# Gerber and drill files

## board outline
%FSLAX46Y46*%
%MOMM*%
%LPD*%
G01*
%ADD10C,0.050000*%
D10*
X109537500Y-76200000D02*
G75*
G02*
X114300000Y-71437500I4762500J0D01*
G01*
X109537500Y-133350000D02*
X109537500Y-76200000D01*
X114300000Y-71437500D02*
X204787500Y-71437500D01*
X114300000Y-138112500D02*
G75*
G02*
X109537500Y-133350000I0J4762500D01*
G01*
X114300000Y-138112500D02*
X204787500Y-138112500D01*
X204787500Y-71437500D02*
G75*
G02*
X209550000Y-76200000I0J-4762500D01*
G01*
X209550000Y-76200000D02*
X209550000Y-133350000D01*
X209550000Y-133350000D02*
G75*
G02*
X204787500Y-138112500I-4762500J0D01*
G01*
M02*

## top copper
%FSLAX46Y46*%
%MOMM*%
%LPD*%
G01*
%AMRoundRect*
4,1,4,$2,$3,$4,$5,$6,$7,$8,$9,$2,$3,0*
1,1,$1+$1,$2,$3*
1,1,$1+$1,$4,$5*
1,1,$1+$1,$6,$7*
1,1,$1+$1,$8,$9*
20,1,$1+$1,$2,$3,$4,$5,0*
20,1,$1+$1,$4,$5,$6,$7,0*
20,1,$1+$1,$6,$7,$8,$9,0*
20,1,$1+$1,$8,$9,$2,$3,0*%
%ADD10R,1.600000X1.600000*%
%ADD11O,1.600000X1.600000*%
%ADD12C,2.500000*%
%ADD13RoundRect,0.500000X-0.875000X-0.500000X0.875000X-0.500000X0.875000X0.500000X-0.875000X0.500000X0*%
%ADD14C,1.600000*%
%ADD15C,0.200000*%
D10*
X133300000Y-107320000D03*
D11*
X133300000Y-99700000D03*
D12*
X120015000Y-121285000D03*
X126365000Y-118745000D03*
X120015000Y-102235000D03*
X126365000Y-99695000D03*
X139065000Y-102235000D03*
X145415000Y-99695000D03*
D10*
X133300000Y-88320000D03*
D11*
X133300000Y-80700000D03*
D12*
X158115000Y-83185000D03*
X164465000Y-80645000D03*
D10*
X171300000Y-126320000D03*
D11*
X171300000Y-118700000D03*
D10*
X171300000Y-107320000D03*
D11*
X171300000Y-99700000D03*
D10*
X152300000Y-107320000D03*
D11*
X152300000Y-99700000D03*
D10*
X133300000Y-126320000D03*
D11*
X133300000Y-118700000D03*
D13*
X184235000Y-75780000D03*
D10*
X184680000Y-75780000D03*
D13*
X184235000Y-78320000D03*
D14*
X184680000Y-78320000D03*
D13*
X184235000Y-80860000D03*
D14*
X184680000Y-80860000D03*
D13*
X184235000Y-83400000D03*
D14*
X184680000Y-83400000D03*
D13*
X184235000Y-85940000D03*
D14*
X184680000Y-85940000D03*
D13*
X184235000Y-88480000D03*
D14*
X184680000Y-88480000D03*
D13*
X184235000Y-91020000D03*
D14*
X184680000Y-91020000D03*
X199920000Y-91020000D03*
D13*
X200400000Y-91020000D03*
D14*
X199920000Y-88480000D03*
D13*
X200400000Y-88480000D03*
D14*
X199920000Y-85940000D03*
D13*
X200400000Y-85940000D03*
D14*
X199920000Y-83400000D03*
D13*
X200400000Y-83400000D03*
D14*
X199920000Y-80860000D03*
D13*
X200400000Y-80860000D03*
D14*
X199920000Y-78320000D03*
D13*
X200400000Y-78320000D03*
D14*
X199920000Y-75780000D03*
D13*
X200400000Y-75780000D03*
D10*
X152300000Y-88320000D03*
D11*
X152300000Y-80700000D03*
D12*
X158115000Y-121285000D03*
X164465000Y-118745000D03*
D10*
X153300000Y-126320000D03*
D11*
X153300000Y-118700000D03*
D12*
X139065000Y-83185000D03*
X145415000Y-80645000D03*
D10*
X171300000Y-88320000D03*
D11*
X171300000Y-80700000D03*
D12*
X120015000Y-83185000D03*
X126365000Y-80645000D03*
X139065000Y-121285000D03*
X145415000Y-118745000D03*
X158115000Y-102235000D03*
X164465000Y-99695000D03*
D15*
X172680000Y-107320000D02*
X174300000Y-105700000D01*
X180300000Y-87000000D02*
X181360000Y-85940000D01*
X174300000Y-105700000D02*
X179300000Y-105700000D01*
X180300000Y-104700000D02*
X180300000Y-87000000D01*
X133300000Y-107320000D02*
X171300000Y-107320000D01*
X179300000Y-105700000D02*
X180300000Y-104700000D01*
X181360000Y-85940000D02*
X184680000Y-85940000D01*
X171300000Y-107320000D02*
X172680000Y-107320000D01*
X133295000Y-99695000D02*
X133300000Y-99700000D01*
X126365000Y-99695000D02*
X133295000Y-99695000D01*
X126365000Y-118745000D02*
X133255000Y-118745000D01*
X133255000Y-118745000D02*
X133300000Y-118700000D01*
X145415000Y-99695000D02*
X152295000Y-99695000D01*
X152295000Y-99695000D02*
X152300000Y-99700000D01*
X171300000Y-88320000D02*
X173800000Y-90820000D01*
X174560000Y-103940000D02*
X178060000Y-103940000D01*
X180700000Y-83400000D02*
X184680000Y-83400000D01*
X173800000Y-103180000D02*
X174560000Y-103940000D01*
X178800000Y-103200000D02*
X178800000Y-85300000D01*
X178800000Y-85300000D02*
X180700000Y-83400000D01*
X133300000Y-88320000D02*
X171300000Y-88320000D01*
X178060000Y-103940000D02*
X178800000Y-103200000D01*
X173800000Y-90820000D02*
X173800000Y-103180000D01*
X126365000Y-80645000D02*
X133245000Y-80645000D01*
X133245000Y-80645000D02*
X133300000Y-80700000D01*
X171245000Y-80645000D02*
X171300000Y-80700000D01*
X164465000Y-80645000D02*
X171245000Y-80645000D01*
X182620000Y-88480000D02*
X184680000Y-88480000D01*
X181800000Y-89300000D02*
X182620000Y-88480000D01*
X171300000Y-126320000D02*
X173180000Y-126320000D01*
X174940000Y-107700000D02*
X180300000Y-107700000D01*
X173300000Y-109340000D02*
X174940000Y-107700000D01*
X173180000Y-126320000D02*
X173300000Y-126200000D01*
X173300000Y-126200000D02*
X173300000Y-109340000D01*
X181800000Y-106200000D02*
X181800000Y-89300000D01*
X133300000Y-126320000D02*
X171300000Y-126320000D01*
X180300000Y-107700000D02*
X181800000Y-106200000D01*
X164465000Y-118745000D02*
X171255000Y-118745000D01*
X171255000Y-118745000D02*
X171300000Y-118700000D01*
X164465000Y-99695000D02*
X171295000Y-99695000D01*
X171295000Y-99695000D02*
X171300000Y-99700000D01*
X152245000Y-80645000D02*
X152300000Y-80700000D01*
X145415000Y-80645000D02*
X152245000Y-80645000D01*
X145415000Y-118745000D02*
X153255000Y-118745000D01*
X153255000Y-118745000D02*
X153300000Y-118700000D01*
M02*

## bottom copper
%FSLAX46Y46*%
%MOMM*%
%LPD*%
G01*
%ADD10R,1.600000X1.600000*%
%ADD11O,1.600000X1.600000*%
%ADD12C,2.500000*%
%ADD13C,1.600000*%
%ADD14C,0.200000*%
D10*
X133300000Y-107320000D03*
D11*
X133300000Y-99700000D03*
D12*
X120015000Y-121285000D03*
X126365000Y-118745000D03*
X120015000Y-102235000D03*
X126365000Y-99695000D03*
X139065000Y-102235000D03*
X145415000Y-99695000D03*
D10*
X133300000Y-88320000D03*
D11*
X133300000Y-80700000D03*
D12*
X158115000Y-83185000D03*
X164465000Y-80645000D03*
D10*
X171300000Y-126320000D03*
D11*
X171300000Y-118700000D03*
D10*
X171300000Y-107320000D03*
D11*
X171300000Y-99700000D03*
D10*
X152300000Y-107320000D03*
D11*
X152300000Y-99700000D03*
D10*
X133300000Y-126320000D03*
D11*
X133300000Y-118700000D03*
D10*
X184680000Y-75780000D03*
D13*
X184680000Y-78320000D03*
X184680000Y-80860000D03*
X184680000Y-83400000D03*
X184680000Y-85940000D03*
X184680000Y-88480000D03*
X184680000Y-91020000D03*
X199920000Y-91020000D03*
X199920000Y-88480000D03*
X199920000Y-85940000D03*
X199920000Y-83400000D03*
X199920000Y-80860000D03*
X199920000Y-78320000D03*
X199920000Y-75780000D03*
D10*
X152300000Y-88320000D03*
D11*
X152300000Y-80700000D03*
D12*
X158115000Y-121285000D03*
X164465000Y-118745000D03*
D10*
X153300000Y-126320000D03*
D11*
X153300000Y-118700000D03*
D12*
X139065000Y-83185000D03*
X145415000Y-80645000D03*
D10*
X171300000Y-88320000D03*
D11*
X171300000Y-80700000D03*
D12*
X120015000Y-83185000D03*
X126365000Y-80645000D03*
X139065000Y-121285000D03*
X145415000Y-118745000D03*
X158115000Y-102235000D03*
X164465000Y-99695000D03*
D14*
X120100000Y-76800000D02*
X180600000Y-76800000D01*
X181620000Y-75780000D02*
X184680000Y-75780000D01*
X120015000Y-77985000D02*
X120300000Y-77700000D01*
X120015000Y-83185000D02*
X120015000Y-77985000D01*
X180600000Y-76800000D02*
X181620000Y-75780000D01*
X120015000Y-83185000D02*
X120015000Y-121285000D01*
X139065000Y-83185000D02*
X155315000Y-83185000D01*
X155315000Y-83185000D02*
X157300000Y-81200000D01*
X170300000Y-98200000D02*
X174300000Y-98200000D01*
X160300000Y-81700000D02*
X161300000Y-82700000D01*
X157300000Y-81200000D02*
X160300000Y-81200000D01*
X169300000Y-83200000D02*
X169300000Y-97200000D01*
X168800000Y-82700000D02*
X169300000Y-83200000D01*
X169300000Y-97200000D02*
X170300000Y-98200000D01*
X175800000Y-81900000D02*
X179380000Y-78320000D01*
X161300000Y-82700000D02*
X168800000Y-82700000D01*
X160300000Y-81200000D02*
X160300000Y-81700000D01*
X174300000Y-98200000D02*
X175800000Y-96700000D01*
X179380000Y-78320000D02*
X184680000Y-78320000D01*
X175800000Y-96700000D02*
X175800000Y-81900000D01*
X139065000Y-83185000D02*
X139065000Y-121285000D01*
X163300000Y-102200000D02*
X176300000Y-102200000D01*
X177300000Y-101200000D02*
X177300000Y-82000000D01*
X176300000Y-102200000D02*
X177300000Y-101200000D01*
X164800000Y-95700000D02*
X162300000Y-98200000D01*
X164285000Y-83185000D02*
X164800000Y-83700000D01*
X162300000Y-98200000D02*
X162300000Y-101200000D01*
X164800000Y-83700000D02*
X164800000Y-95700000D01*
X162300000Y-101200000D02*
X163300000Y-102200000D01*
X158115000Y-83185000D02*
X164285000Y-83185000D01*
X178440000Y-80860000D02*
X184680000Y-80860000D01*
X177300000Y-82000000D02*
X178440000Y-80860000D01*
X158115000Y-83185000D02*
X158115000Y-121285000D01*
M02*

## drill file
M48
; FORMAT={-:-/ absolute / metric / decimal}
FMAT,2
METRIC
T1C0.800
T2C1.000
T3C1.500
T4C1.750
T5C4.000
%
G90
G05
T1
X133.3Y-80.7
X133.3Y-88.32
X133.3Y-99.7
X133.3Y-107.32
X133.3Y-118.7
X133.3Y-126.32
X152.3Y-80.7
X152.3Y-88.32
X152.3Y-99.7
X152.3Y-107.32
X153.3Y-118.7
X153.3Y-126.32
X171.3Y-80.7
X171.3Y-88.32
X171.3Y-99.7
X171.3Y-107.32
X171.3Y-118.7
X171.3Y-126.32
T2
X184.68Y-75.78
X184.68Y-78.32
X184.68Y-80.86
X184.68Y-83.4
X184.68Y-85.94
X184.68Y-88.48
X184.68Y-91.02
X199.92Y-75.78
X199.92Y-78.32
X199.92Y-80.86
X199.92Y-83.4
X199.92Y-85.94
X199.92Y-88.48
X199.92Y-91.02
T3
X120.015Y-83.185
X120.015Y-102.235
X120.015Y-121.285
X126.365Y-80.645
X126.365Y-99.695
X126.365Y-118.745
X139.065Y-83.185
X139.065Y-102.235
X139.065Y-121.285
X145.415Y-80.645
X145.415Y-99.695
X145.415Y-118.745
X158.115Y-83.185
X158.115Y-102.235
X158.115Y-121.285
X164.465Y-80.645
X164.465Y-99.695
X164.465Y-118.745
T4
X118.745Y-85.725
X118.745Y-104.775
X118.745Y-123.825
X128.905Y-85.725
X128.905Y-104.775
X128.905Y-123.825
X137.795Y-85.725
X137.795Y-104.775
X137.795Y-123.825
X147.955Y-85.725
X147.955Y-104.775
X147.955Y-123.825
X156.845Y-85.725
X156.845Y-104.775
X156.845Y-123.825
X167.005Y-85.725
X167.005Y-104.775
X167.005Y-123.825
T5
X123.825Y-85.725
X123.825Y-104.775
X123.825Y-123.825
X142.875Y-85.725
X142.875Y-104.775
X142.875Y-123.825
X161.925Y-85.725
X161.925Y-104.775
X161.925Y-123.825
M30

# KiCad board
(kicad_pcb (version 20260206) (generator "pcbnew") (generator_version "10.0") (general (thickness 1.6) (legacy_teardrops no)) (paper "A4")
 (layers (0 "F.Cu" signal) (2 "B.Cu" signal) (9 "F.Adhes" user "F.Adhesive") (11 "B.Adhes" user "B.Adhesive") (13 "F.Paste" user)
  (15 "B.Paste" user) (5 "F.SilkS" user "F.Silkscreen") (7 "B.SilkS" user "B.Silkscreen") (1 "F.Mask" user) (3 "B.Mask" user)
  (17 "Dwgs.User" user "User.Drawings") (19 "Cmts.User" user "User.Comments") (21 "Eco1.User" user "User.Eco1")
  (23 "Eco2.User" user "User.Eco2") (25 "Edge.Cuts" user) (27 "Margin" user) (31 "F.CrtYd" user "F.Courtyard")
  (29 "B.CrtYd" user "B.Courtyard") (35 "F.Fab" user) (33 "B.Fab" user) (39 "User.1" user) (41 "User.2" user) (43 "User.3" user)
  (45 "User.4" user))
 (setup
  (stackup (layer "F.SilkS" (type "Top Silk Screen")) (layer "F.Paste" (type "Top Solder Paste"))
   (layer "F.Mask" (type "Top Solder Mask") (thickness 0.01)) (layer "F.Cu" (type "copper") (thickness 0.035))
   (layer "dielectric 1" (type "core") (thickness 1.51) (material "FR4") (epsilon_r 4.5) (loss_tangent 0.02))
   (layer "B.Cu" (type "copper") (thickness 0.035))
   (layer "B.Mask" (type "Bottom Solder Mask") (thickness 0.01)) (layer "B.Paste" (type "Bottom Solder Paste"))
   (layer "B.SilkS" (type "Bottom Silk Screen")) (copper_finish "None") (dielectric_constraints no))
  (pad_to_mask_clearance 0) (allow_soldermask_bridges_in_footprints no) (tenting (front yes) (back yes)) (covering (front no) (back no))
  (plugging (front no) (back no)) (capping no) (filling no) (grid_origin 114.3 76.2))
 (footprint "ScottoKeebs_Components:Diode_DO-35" (layer "F.Cu") (at 133.3 107.32 90)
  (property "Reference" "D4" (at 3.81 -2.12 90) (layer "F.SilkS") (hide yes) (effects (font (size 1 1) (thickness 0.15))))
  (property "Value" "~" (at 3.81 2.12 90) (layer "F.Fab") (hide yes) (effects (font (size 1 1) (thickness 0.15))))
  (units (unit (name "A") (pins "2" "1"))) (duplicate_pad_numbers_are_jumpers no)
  (pad "1" thru_hole rect (at 0 0 90) (size 1.6 1.6) (drill 0.8) (layers "*.Cu" "*.Mask") (remove_unused_layers no) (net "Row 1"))
  (pad "2" thru_hole oval (at 7.62 0 90) (size 1.6 1.6) (drill 0.8) (layers "*.Cu" "*.Mask") (remove_unused_layers no) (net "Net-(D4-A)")))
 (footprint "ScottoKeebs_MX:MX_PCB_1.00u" (layer "F.Cu") (at 123.825 123.825)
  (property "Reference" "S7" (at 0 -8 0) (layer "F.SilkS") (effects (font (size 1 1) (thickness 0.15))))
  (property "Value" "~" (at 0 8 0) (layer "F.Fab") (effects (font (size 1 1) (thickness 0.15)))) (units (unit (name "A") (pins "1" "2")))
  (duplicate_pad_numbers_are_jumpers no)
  (pad "" np_thru_hole circle (at -5.08 0) (size 1.75 1.75) (drill 1.75) (layers "*.Cu" "*.Mask"))
  (pad "" np_thru_hole circle (at 0 0) (size 4 4) (drill 4) (layers "*.Cu" "*.Mask"))
  (pad "" np_thru_hole circle (at 5.08 0) (size 1.75 1.75) (drill 1.75) (layers "*.Cu" "*.Mask"))
  (pad "1" thru_hole circle (at -3.81 -2.54) (size 2.5 2.5) (drill 1.5) (layers "*.Cu" "*.Mask") (remove_unused_layers no) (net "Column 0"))
  (pad "2" thru_hole circle (at 2.54 -5.08) (size 2.5 2.5) (drill 1.5) (layers "*.Cu" "*.Mask") (remove_unused_layers no) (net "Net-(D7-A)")))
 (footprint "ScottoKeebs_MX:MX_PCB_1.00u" (layer "F.Cu") (at 123.825 104.775)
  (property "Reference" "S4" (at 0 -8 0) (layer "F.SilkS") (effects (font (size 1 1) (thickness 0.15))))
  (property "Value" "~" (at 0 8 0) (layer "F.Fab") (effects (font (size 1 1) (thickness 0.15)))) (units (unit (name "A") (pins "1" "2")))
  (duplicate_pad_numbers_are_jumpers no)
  (pad "" np_thru_hole circle (at -5.08 0) (size 1.75 1.75) (drill 1.75) (layers "*.Cu" "*.Mask"))
  (pad "" np_thru_hole circle (at 0 0) (size 4 4) (drill 4) (layers "*.Cu" "*.Mask"))
  (pad "" np_thru_hole circle (at 5.08 0) (size 1.75 1.75) (drill 1.75) (layers "*.Cu" "*.Mask"))
  (pad "1" thru_hole circle (at -3.81 -2.54) (size 2.5 2.5) (drill 1.5) (layers "*.Cu" "*.Mask") (remove_unused_layers no) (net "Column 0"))
  (pad "2" thru_hole circle (at 2.54 -5.08) (size 2.5 2.5) (drill 1.5) (layers "*.Cu" "*.Mask") (remove_unused_layers no) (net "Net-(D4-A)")))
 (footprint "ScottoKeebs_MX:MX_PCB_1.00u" (layer "F.Cu") (at 142.875 104.775)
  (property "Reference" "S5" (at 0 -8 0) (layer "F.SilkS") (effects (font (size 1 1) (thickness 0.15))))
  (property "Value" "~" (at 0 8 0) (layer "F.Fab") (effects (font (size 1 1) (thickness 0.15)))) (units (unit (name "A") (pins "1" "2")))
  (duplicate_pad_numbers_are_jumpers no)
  (pad "" np_thru_hole circle (at -5.08 0) (size 1.75 1.75) (drill 1.75) (layers "*.Cu" "*.Mask"))
  (pad "" np_thru_hole circle (at 0 0) (size 4 4) (drill 4) (layers "*.Cu" "*.Mask"))
  (pad "" np_thru_hole circle (at 5.08 0) (size 1.75 1.75) (drill 1.75) (layers "*.Cu" "*.Mask"))
  (pad "1" thru_hole circle (at -3.81 -2.54) (size 2.5 2.5) (drill 1.5) (layers "*.Cu" "*.Mask") (remove_unused_layers no) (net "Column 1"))
  (pad "2" thru_hole circle (at 2.54 -5.08) (size 2.5 2.5) (drill 1.5) (layers "*.Cu" "*.Mask") (remove_unused_layers no) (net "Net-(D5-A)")))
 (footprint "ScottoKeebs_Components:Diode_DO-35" (layer "F.Cu") (at 133.3 88.32 90)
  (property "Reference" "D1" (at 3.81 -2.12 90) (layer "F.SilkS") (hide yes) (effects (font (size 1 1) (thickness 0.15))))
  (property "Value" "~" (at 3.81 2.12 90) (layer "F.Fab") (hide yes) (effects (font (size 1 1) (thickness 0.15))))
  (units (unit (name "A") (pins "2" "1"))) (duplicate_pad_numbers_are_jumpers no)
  (pad "1" thru_hole rect (at 0 0 90) (size 1.6 1.6) (drill 0.8) (layers "*.Cu" "*.Mask") (remove_unused_layers no) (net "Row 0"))
  (pad "2" thru_hole oval (at 7.62 0 90) (size 1.6 1.6) (drill 0.8) (layers "*.Cu" "*.Mask") (remove_unused_layers no) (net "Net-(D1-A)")))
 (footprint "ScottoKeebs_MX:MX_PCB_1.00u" (layer "F.Cu") (at 161.925 85.725)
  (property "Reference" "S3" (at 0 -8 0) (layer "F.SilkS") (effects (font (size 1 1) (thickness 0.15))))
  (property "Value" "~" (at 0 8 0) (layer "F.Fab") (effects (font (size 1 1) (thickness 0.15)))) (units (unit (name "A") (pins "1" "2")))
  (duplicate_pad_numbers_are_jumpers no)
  (pad "" np_thru_hole circle (at -5.08 0) (size 1.75 1.75) (drill 1.75) (layers "*.Cu" "*.Mask"))
  (pad "" np_thru_hole circle (at 0 0) (size 4 4) (drill 4) (layers "*.Cu" "*.Mask"))
  (pad "" np_thru_hole circle (at 5.08 0) (size 1.75 1.75) (drill 1.75) (layers "*.Cu" "*.Mask"))
  (pad "1" thru_hole circle (at -3.81 -2.54) (size 2.5 2.5) (drill 1.5) (layers "*.Cu" "*.Mask") (remove_unused_layers no) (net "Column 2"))
  (pad "2" thru_hole circle (at 2.54 -5.08) (size 2.5 2.5) (drill 1.5) (layers "*.Cu" "*.Mask") (remove_unused_layers no) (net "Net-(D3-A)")))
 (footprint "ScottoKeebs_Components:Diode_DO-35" (layer "F.Cu") (at 171.3 126.32 90)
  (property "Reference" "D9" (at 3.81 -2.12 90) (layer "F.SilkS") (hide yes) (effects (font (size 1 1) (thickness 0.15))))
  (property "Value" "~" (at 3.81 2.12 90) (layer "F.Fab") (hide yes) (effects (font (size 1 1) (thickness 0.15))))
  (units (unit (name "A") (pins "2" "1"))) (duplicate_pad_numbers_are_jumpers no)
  (pad "1" thru_hole rect (at 0 0 90) (size 1.6 1.6) (drill 0.8) (layers "*.Cu" "*.Mask") (remove_unused_layers no) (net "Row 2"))
  (pad "2" thru_hole oval (at 7.62 0 90) (size 1.6 1.6) (drill 0.8) (layers "*.Cu" "*.Mask") (remove_unused_layers no) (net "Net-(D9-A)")))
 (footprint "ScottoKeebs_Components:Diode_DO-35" (layer "F.Cu") (at 171.3 107.32 90)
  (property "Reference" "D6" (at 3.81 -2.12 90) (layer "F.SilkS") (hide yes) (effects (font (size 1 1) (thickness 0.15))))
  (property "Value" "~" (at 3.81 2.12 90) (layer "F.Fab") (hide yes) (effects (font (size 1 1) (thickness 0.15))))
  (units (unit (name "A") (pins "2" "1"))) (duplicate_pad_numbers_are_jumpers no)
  (pad "1" thru_hole rect (at 0 0 90) (size 1.6 1.6) (drill 0.8) (layers "*.Cu" "*.Mask") (remove_unused_layers no) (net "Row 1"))
  (pad "2" thru_hole oval (at 7.62 0 90) (size 1.6 1.6) (drill 0.8) (layers "*.Cu" "*.Mask") (remove_unused_layers no) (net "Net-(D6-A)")))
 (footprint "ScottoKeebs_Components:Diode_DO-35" (layer "F.Cu") (at 152.3 107.32 90)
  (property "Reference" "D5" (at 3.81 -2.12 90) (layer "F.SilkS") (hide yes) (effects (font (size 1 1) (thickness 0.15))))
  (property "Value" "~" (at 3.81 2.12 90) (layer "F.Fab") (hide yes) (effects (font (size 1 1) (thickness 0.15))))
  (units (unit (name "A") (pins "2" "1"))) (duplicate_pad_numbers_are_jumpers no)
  (pad "1" thru_hole rect (at 0 0 90) (size 1.6 1.6) (drill 0.8) (layers "*.Cu" "*.Mask") (remove_unused_layers no) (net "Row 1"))
  (pad "2" thru_hole oval (at 7.62 0 90) (size 1.6 1.6) (drill 0.8) (layers "*.Cu" "*.Mask") (remove_unused_layers no) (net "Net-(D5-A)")))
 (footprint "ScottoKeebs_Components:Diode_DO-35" (layer "F.Cu") (at 133.3 126.32 90)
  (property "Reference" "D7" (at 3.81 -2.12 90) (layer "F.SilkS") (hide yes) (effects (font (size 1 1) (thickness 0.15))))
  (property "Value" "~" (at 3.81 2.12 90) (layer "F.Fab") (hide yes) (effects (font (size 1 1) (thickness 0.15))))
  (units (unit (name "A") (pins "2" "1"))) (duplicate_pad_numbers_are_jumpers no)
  (pad "1" thru_hole rect (at 0 0 90) (size 1.6 1.6) (drill 0.8) (layers "*.Cu" "*.Mask") (remove_unused_layers no) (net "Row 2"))
  (pad "2" thru_hole oval (at 7.62 0 90) (size 1.6 1.6) (drill 0.8) (layers "*.Cu" "*.Mask") (remove_unused_layers no) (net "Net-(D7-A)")))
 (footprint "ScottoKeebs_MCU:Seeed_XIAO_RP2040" (layer "F.Cu") (at 192.3 83.4)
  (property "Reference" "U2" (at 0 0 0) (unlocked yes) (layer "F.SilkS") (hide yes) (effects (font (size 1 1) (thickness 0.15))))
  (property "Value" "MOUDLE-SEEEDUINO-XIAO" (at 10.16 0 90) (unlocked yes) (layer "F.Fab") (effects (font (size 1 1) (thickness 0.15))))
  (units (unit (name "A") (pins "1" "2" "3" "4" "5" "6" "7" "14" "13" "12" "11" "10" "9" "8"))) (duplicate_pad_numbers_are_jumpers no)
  (pad "1" smd roundrect (at -8.065 -7.62) (size 2.75 2) (layers "F.Cu" "F.Mask" "F.Paste") (roundrect_rratio 0.25) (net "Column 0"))
  (pad "1" thru_hole rect (at -7.62 -7.62 90) (size 1.6 1.6) (drill 1) (layers "*.Cu" "*.Mask") (remove_unused_layers no) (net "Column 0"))
  (pad "2" smd roundrect (at -8.065 -5.08) (size 2.75 2) (layers "F.Cu" "F.Mask" "F.Paste") (roundrect_rratio 0.25) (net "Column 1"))
  (pad "2" thru_hole circle (at -7.62 -5.08 90) (size 1.6 1.6) (drill 1) (layers "*.Cu" "*.Mask") (remove_unused_layers no) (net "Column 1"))
  (pad "3" smd roundrect (at -8.065 -2.54) (size 2.75 2) (layers "F.Cu" "F.Mask" "F.Paste") (roundrect_rratio 0.25) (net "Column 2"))
  (pad "3" thru_hole circle (at -7.62 -2.54 90) (size 1.6 1.6) (drill 1) (layers "*.Cu" "*.Mask") (remove_unused_layers no) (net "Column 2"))
  (pad "4" smd roundrect (at -8.065 0) (size 2.75 2) (layers "F.Cu" "F.Mask" "F.Paste") (roundrect_rratio 0.25) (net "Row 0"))
  (pad "4" thru_hole circle (at -7.62 0 90) (size 1.6 1.6) (drill 1) (layers "*.Cu" "*.Mask") (remove_unused_layers no) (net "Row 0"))
  (pad "5" smd roundrect (at -8.065 2.54) (size 2.75 2) (layers "F.Cu" "F.Mask" "F.Paste") (roundrect_rratio 0.25) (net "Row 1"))
  (pad "5" thru_hole circle (at -7.62 2.54 90) (size 1.6 1.6) (drill 1) (layers "*.Cu" "*.Mask") (remove_unused_layers no) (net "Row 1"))
  (pad "6" smd roundrect (at -8.065 5.08) (size 2.75 2) (layers "F.Cu" "F.Mask" "F.Paste") (roundrect_rratio 0.25) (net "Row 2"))
  (pad "6" thru_hole circle (at -7.62 5.08 90) (size 1.6 1.6) (drill 1) (layers "*.Cu" "*.Mask") (remove_unused_layers no) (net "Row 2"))
  (pad "7" smd roundrect (at -8.065 7.62) (size 2.75 2) (layers "F.Cu" "F.Mask" "F.Paste") (roundrect_rratio 0.25)
   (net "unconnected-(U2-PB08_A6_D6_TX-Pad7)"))
  (pad "7" thru_hole circle (at -7.62 7.62 90) (size 1.6 1.6) (drill 1) (layers "*.Cu" "*.Mask") (remove_unused_layers no)
   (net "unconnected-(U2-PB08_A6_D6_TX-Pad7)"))
  (pad "8" thru_hole circle (at 7.62 7.62 90) (size 1.6 1.6) (drill 1) (layers "*.Cu" "*.Mask") (remove_unused_layers no)
   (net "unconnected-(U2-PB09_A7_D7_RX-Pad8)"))
  (pad "8" smd roundrect (at 8.1 7.62) (size 2.75 2) (layers "F.Cu" "F.Mask" "F.Paste") (roundrect_rratio 0.25)
   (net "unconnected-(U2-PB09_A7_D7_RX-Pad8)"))
  (pad "9" thru_hole circle (at 7.62 5.08 90) (size 1.6 1.6) (drill 1) (layers "*.Cu" "*.Mask") (remove_unused_layers no)
   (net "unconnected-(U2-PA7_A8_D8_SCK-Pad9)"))
  (pad "9" smd roundrect (at 8.1 5.08) (size 2.75 2) (layers "F.Cu" "F.Mask" "F.Paste") (roundrect_rratio 0.25)
   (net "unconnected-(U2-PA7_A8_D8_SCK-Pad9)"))
  (pad "10" thru_hole circle (at 7.62 2.54 90) (size 1.6 1.6) (drill 1) (layers "*.Cu" "*.Mask") (remove_unused_layers no)
   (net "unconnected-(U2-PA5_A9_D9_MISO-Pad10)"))
  (pad "10" smd roundrect (at 8.1 2.54) (size 2.75 2) (layers "F.Cu" "F.Mask" "F.Paste") (roundrect_rratio 0.25)
   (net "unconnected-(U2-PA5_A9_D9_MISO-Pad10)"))
  (pad "11" thru_hole circle (at 7.62 0 90) (size 1.6 1.6) (drill 1) (layers "*.Cu" "*.Mask") (remove_unused_layers no)
   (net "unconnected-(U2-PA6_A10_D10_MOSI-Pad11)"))
  (pad "11" smd roundrect (at 8.1 0) (size 2.75 2) (layers "F.Cu" "F.Mask" "F.Paste") (roundrect_rratio 0.25)
   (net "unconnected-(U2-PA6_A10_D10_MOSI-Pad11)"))
  (pad "12" thru_hole circle (at 7.62 -2.54 90) (size 1.6 1.6) (drill 1) (layers "*.Cu" "*.Mask") (remove_unused_layers no)
   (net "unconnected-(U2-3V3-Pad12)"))
  (pad "12" smd roundrect (at 8.1 -2.54) (size 2.75 2) (layers "F.Cu" "F.Mask" "F.Paste") (roundrect_rratio 0.25)
   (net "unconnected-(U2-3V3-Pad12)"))
  (pad "13" thru_hole circle (at 7.62 -5.08 90) (size 1.6 1.6) (drill 1) (layers "*.Cu" "*.Mask") (remove_unused_layers no)
   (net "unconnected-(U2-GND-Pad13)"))
  (pad "13" smd roundrect (at 8.1 -5.08) (size 2.75 2) (layers "F.Cu" "F.Mask" "F.Paste") (roundrect_rratio 0.25)
   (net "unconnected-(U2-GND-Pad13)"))
  (pad "14" thru_hole circle (at 7.62 -7.62 90) (size 1.6 1.6) (drill 1) (layers "*.Cu" "*.Mask") (remove_unused_layers no)
   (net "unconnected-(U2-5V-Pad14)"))
  (pad "14" smd roundrect (at 8.1 -7.62) (size 2.75 2) (layers "F.Cu" "F.Mask" "F.Paste") (roundrect_rratio 0.25)
   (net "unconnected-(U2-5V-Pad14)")))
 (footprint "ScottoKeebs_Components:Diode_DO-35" (layer "F.Cu") (at 152.3 88.32 90)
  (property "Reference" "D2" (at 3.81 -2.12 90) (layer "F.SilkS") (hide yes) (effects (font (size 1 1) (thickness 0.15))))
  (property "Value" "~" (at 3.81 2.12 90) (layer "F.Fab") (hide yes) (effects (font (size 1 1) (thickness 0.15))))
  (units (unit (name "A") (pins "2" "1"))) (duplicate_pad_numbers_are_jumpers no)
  (pad "1" thru_hole rect (at 0 0 90) (size 1.6 1.6) (drill 0.8) (layers "*.Cu" "*.Mask") (remove_unused_layers no) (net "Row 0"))
  (pad "2" thru_hole oval (at 7.62 0 90) (size 1.6 1.6) (drill 0.8) (layers "*.Cu" "*.Mask") (remove_unused_layers no) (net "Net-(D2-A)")))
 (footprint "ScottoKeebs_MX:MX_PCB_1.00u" (layer "F.Cu") (at 161.925 123.825)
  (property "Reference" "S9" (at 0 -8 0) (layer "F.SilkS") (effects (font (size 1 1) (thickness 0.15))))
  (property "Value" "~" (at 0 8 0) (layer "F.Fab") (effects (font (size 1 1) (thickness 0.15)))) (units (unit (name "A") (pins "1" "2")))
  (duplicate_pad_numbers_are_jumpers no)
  (pad "" np_thru_hole circle (at -5.08 0) (size 1.75 1.75) (drill 1.75) (layers "*.Cu" "*.Mask"))
  (pad "" np_thru_hole circle (at 0 0) (size 4 4) (drill 4) (layers "*.Cu" "*.Mask"))
  (pad "" np_thru_hole circle (at 5.08 0) (size 1.75 1.75) (drill 1.75) (layers "*.Cu" "*.Mask"))
  (pad "1" thru_hole circle (at -3.81 -2.54) (size 2.5 2.5) (drill 1.5) (layers "*.Cu" "*.Mask") (remove_unused_layers no) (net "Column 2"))
  (pad "2" thru_hole circle (at 2.54 -5.08) (size 2.5 2.5) (drill 1.5) (layers "*.Cu" "*.Mask") (remove_unused_layers no) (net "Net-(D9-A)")))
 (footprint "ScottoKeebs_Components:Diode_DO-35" (layer "F.Cu") (at 153.3 126.32 90)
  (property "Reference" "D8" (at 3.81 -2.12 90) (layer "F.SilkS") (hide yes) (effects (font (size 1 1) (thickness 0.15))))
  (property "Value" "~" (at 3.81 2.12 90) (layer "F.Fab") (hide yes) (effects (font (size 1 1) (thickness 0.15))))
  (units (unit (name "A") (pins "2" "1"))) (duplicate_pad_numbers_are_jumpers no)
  (pad "1" thru_hole rect (at 0 0 90) (size 1.6 1.6) (drill 0.8) (layers "*.Cu" "*.Mask") (remove_unused_layers no) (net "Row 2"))
  (pad "2" thru_hole oval (at 7.62 0 90) (size 1.6 1.6) (drill 0.8) (layers "*.Cu" "*.Mask") (remove_unused_layers no) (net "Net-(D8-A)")))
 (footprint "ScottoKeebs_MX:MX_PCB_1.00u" (layer "F.Cu") (at 142.875 85.725)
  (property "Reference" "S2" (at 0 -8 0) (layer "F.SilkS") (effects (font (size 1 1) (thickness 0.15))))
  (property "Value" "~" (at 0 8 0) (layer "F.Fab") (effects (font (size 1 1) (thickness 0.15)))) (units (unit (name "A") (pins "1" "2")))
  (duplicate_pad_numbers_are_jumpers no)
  (pad "" np_thru_hole circle (at -5.08 0) (size 1.75 1.75) (drill 1.75) (layers "*.Cu" "*.Mask"))
  (pad "" np_thru_hole circle (at 0 0) (size 4 4) (drill 4) (layers "*.Cu" "*.Mask"))
  (pad "" np_thru_hole circle (at 5.08 0) (size 1.75 1.75) (drill 1.75) (layers "*.Cu" "*.Mask"))
  (pad "1" thru_hole circle (at -3.81 -2.54) (size 2.5 2.5) (drill 1.5) (layers "*.Cu" "*.Mask") (remove_unused_layers no) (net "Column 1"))
  (pad "2" thru_hole circle (at 2.54 -5.08) (size 2.5 2.5) (drill 1.5) (layers "*.Cu" "*.Mask") (remove_unused_layers no) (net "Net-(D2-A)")))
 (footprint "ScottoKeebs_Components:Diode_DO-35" (layer "F.Cu") (at 171.3 88.32 90)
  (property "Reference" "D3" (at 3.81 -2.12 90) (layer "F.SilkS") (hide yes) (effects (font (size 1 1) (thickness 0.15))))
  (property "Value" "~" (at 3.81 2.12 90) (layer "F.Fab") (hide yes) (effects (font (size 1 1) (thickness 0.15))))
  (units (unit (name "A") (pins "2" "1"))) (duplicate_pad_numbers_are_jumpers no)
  (pad "1" thru_hole rect (at 0 0 90) (size 1.6 1.6) (drill 0.8) (layers "*.Cu" "*.Mask") (remove_unused_layers no) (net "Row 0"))
  (pad "2" thru_hole oval (at 7.62 0 90) (size 1.6 1.6) (drill 0.8) (layers "*.Cu" "*.Mask") (remove_unused_layers no) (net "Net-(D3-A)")))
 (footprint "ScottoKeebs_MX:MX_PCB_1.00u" (layer "F.Cu") (at 123.825 85.725)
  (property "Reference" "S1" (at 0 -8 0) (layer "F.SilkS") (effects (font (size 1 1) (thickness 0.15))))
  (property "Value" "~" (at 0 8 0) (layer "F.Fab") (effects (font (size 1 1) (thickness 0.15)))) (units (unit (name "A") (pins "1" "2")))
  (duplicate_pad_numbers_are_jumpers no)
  (pad "" np_thru_hole circle (at -5.08 0) (size 1.75 1.75) (drill 1.75) (layers "*.Cu" "*.Mask"))
  (pad "" np_thru_hole circle (at 0 0) (size 4 4) (drill 4) (layers "*.Cu" "*.Mask"))
  (pad "" np_thru_hole circle (at 5.08 0) (size 1.75 1.75) (drill 1.75) (layers "*.Cu" "*.Mask"))
  (pad "1" thru_hole circle (at -3.81 -2.54) (size 2.5 2.5) (drill 1.5) (layers "*.Cu" "*.Mask") (remove_unused_layers no) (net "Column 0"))
  (pad "2" thru_hole circle (at 2.54 -5.08) (size 2.5 2.5) (drill 1.5) (layers "*.Cu" "*.Mask") (remove_unused_layers no) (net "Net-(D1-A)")))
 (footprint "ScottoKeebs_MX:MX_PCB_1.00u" (layer "F.Cu") (at 142.875 123.825)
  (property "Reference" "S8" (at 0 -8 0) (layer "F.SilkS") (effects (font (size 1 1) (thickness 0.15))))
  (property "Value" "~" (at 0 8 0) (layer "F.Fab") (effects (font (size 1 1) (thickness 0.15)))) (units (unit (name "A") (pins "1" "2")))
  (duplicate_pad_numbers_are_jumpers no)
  (pad "" np_thru_hole circle (at -5.08 0) (size 1.75 1.75) (drill 1.75) (layers "*.Cu" "*.Mask"))
  (pad "" np_thru_hole circle (at 0 0) (size 4 4) (drill 4) (layers "*.Cu" "*.Mask"))
  (pad "" np_thru_hole circle (at 5.08 0) (size 1.75 1.75) (drill 1.75) (layers "*.Cu" "*.Mask"))
  (pad "1" thru_hole circle (at -3.81 -2.54) (size 2.5 2.5) (drill 1.5) (layers "*.Cu" "*.Mask") (remove_unused_layers no) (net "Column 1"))
  (pad "2" thru_hole circle (at 2.54 -5.08) (size 2.5 2.5) (drill 1.5) (layers "*.Cu" "*.Mask") (remove_unused_layers no) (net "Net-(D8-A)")))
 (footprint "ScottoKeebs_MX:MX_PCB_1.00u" (layer "F.Cu") (at 161.925 104.775)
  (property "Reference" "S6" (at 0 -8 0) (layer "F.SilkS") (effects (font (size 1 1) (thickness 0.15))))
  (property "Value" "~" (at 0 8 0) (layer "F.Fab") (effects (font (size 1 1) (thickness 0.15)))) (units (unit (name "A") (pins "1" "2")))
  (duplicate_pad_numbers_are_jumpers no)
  (pad "" np_thru_hole circle (at -5.08 0) (size 1.75 1.75) (drill 1.75) (layers "*.Cu" "*.Mask"))
  (pad "" np_thru_hole circle (at 0 0) (size 4 4) (drill 4) (layers "*.Cu" "*.Mask"))
  (pad "" np_thru_hole circle (at 5.08 0) (size 1.75 1.75) (drill 1.75) (layers "*.Cu" "*.Mask"))
  (pad "1" thru_hole circle (at -3.81 -2.54) (size 2.5 2.5) (drill 1.5) (layers "*.Cu" "*.Mask") (remove_unused_layers no) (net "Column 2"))
  (pad "2" thru_hole circle (at 2.54 -5.08) (size 2.5 2.5) (drill 1.5) (layers "*.Cu" "*.Mask") (remove_unused_layers no) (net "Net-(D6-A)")))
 (gr_arc (start 109.5375 76.2) (mid 110.932404 72.832404) (end 114.3 71.4375) (stroke (width 0.05) (type default)) (layer "Edge.Cuts"))
 (gr_line (start 109.5375 133.35) (end 109.5375 76.2) (stroke (width 0.05) (type default)) (layer "Edge.Cuts"))
 (gr_line (start 114.3 71.4375) (end 204.7875 71.4375) (stroke (width 0.05) (type default)) (layer "Edge.Cuts"))
 (gr_arc (start 114.3 138.1125) (mid 110.932404 136.717596) (end 109.5375 133.35) (stroke (width 0.05) (type default)) (layer "Edge.Cuts"))
 (gr_line (start 114.3 138.1125) (end 204.7875 138.1125) (stroke (width 0.05) (type default)) (layer "Edge.Cuts"))
 (gr_arc (start 204.7875 71.4375) (mid 208.155096 72.832404) (end 209.55 76.2) (stroke (width 0.05) (type default)) (layer "Edge.Cuts"))
 (gr_line (start 209.55 76.2) (end 209.55 133.35) (stroke (width 0.05) (type default)) (layer "Edge.Cuts"))
 (gr_arc (start 209.55 133.35) (mid 208.155096 136.717596) (end 204.7875 138.1125) (stroke (width 0.05) (type default)) (layer "Edge.Cuts"))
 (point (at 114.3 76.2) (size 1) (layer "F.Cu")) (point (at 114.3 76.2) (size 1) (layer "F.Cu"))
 (segment (start 172.68 107.32) (end 174.3 105.7) (width 0.2) (layer "F.Cu") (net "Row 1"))
 (segment (start 180.3 87) (end 181.36 85.94) (width 0.2) (layer "F.Cu") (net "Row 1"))
 (segment (start 174.3 105.7) (end 179.3 105.7) (width 0.2) (layer "F.Cu") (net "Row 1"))
 (segment (start 180.3 104.7) (end 180.3 87) (width 0.2) (layer "F.Cu") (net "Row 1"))
 (segment (start 133.3 107.32) (end 171.3 107.32) (width 0.2) (layer "F.Cu") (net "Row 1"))
 (segment (start 179.3 105.7) (end 180.3 104.7) (width 0.2) (layer "F.Cu") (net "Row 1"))
 (segment (start 181.36 85.94) (end 184.68 85.94) (width 0.2) (layer "F.Cu") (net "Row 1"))
 (segment (start 171.3 107.32) (end 172.68 107.32) (width 0.2) (layer "F.Cu") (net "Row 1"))
 (segment (start 133.295 99.695) (end 133.3 99.7) (width 0.2) (layer "F.Cu") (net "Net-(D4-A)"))
 (segment (start 126.365 99.695) (end 133.295 99.695) (width 0.2) (layer "F.Cu") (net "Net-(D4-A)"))
 (segment (start 120.1 76.8) (end 180.6 76.8) (width 0.2) (layer "B.Cu") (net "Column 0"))
 (segment (start 181.62 75.78) (end 184.68 75.78) (width 0.2) (layer "B.Cu") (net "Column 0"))
 (segment (start 120.015 77.985) (end 120.3 77.7) (width 0.2) (layer "B.Cu") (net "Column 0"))
 (segment (start 120.015 83.185) (end 120.015 77.985) (width 0.2) (layer "B.Cu") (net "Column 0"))
 (segment (start 180.6 76.8) (end 181.62 75.78) (width 0.2) (layer "B.Cu") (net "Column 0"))
 (segment (start 120.015 83.185) (end 120.015 121.285) (width 0.2) (layer "B.Cu") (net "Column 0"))
 (segment (start 126.365 118.745) (end 133.255 118.745) (width 0.2) (layer "F.Cu") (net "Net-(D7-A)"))
 (segment (start 133.255 118.745) (end 133.3 118.7) (width 0.2) (layer "F.Cu") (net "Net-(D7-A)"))
 (segment (start 139.065 83.185) (end 155.315 83.185) (width 0.2) (layer "B.Cu") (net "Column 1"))
 (segment (start 155.315 83.185) (end 157.3 81.2) (width 0.2) (layer "B.Cu") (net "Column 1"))
 (segment (start 170.3 98.2) (end 174.3 98.2) (width 0.2) (layer "B.Cu") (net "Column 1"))
 (segment (start 160.3 81.7) (end 161.3 82.7) (width 0.2) (layer "B.Cu") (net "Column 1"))
 (segment (start 157.3 81.2) (end 160.3 81.2) (width 0.2) (layer "B.Cu") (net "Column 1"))
 (segment (start 169.3 83.2) (end 169.3 97.2) (width 0.2) (layer "B.Cu") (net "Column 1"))
 (segment (start 168.8 82.7) (end 169.3 83.2) (width 0.2) (layer "B.Cu") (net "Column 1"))
 (segment (start 169.3 97.2) (end 170.3 98.2) (width 0.2) (layer "B.Cu") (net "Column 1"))
 (segment (start 175.8 81.9) (end 179.38 78.32) (width 0.2) (layer "B.Cu") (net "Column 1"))
 (segment (start 161.3 82.7) (end 168.8 82.7) (width 0.2) (layer "B.Cu") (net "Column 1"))
 (segment (start 160.3 81.2) (end 160.3 81.7) (width 0.2) (layer "B.Cu") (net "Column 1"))
 (segment (start 174.3 98.2) (end 175.8 96.7) (width 0.2) (layer "B.Cu") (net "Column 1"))
 (segment (start 179.38 78.32) (end 184.68 78.32) (width 0.2) (layer "B.Cu") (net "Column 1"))
 (segment (start 175.8 96.7) (end 175.8 81.9) (width 0.2) (layer "B.Cu") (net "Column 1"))
 (segment (start 139.065 83.185) (end 139.065 121.285) (width 0.2) (layer "B.Cu") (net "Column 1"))
 (segment (start 145.415 99.695) (end 152.295 99.695) (width 0.2) (layer "F.Cu") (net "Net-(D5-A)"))
 (segment (start 152.295 99.695) (end 152.3 99.7) (width 0.2) (layer "F.Cu") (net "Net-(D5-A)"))
 (segment (start 171.3 88.32) (end 173.8 90.82) (width 0.2) (layer "F.Cu") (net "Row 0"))
 (segment (start 174.56 103.94) (end 178.06 103.94) (width 0.2) (layer "F.Cu") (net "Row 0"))
 (segment (start 180.7 83.4) (end 184.68 83.4) (width 0.2) (layer "F.Cu") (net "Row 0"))
 (segment (start 173.8 103.18) (end 174.56 103.94) (width 0.2) (layer "F.Cu") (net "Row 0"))
 (segment (start 178.8 103.2) (end 178.8 85.3) (width 0.2) (layer "F.Cu") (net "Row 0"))
 (segment (start 178.8 85.3) (end 180.7 83.4) (width 0.2) (layer "F.Cu") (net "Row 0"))
 (segment (start 133.3 88.32) (end 171.3 88.32) (width 0.2) (layer "F.Cu") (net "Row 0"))
 (segment (start 178.06 103.94) (end 178.8 103.2) (width 0.2) (layer "F.Cu") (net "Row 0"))
 (segment (start 173.8 90.82) (end 173.8 103.18) (width 0.2) (layer "F.Cu") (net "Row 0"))
 (segment (start 126.365 80.645) (end 133.245 80.645) (width 0.2) (layer "F.Cu") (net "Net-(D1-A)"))
 (segment (start 133.245 80.645) (end 133.3 80.7) (width 0.2) (layer "F.Cu") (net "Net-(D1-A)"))
 (segment (start 163.3 102.2) (end 176.3 102.2) (width 0.2) (layer "B.Cu") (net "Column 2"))
 (segment (start 177.3 101.2) (end 177.3 82) (width 0.2) (layer "B.Cu") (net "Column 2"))
 (segment (start 176.3 102.2) (end 177.3 101.2) (width 0.2) (layer "B.Cu") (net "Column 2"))
 (segment (start 164.8 95.7) (end 162.3 98.2) (width 0.2) (layer "B.Cu") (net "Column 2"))
 (segment (start 164.285 83.185) (end 164.8 83.7) (width 0.2) (layer "B.Cu") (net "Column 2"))
 (segment (start 162.3 98.2) (end 162.3 101.2) (width 0.2) (layer "B.Cu") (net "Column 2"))
 (segment (start 164.8 83.7) (end 164.8 95.7) (width 0.2) (layer "B.Cu") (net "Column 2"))
 (segment (start 162.3 101.2) (end 163.3 102.2) (width 0.2) (layer "B.Cu") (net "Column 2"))
 (segment (start 158.115 83.185) (end 164.285 83.185) (width 0.2) (layer "B.Cu") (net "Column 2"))
 (segment (start 178.44 80.86) (end 184.68 80.86) (width 0.2) (layer "B.Cu") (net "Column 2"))
 (segment (start 177.3 82) (end 178.44 80.86) (width 0.2) (layer "B.Cu") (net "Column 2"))
 (segment (start 158.115 83.185) (end 158.115 121.285) (width 0.2) (layer "B.Cu") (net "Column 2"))
 (segment (start 171.245 80.645) (end 171.3 80.7) (width 0.2) (layer "F.Cu") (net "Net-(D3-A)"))
 (segment (start 164.465 80.645) (end 171.245 80.645) (width 0.2) (layer "F.Cu") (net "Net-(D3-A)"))
 (segment (start 182.62 88.48) (end 184.68 88.48) (width 0.2) (layer "F.Cu") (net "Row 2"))
 (segment (start 181.8 89.3) (end 182.62 88.48) (width 0.2) (layer "F.Cu") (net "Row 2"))
 (segment (start 171.3 126.32) (end 173.18 126.32) (width 0.2) (layer "F.Cu") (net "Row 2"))
 (segment (start 174.94 107.7) (end 180.3 107.7) (width 0.2) (layer "F.Cu") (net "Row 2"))
 (segment (start 173.3 109.34) (end 174.94 107.7) (width 0.2) (layer "F.Cu") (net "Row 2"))
 (segment (start 173.18 126.32) (end 173.3 126.2) (width 0.2) (layer "F.Cu") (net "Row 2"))
 (segment (start 173.3 126.2) (end 173.3 109.34) (width 0.2) (layer "F.Cu") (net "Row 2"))
 (segment (start 181.8 106.2) (end 181.8 89.3) (width 0.2) (layer "F.Cu") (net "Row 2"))
 (segment (start 133.3 126.32) (end 171.3 126.32) (width 0.2) (layer "F.Cu") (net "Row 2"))
 (segment (start 180.3 107.7) (end 181.8 106.2) (width 0.2) (layer "F.Cu") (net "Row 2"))
 (segment (start 164.465 118.745) (end 171.255 118.745) (width 0.2) (layer "F.Cu") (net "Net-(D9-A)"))
 (segment (start 171.255 118.745) (end 171.3 118.7) (width 0.2) (layer "F.Cu") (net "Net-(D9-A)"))
 (segment (start 164.465 99.695) (end 171.295 99.695) (width 0.2) (layer "F.Cu") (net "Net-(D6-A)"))
 (segment (start 171.295 99.695) (end 171.3 99.7) (width 0.2) (layer "F.Cu") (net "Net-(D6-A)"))
 (segment (start 152.245 80.645) (end 152.3 80.7) (width 0.2) (layer "F.Cu") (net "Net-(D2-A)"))
 (segment (start 145.415 80.645) (end 152.245 80.645) (width 0.2) (layer "F.Cu") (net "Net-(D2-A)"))
 (segment (start 145.415 118.745) (end 153.255 118.745) (width 0.2) (layer "F.Cu") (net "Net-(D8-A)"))
 (segment (start 153.255 118.745) (end 153.3 118.7) (width 0.2) (layer "F.Cu") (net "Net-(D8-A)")))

